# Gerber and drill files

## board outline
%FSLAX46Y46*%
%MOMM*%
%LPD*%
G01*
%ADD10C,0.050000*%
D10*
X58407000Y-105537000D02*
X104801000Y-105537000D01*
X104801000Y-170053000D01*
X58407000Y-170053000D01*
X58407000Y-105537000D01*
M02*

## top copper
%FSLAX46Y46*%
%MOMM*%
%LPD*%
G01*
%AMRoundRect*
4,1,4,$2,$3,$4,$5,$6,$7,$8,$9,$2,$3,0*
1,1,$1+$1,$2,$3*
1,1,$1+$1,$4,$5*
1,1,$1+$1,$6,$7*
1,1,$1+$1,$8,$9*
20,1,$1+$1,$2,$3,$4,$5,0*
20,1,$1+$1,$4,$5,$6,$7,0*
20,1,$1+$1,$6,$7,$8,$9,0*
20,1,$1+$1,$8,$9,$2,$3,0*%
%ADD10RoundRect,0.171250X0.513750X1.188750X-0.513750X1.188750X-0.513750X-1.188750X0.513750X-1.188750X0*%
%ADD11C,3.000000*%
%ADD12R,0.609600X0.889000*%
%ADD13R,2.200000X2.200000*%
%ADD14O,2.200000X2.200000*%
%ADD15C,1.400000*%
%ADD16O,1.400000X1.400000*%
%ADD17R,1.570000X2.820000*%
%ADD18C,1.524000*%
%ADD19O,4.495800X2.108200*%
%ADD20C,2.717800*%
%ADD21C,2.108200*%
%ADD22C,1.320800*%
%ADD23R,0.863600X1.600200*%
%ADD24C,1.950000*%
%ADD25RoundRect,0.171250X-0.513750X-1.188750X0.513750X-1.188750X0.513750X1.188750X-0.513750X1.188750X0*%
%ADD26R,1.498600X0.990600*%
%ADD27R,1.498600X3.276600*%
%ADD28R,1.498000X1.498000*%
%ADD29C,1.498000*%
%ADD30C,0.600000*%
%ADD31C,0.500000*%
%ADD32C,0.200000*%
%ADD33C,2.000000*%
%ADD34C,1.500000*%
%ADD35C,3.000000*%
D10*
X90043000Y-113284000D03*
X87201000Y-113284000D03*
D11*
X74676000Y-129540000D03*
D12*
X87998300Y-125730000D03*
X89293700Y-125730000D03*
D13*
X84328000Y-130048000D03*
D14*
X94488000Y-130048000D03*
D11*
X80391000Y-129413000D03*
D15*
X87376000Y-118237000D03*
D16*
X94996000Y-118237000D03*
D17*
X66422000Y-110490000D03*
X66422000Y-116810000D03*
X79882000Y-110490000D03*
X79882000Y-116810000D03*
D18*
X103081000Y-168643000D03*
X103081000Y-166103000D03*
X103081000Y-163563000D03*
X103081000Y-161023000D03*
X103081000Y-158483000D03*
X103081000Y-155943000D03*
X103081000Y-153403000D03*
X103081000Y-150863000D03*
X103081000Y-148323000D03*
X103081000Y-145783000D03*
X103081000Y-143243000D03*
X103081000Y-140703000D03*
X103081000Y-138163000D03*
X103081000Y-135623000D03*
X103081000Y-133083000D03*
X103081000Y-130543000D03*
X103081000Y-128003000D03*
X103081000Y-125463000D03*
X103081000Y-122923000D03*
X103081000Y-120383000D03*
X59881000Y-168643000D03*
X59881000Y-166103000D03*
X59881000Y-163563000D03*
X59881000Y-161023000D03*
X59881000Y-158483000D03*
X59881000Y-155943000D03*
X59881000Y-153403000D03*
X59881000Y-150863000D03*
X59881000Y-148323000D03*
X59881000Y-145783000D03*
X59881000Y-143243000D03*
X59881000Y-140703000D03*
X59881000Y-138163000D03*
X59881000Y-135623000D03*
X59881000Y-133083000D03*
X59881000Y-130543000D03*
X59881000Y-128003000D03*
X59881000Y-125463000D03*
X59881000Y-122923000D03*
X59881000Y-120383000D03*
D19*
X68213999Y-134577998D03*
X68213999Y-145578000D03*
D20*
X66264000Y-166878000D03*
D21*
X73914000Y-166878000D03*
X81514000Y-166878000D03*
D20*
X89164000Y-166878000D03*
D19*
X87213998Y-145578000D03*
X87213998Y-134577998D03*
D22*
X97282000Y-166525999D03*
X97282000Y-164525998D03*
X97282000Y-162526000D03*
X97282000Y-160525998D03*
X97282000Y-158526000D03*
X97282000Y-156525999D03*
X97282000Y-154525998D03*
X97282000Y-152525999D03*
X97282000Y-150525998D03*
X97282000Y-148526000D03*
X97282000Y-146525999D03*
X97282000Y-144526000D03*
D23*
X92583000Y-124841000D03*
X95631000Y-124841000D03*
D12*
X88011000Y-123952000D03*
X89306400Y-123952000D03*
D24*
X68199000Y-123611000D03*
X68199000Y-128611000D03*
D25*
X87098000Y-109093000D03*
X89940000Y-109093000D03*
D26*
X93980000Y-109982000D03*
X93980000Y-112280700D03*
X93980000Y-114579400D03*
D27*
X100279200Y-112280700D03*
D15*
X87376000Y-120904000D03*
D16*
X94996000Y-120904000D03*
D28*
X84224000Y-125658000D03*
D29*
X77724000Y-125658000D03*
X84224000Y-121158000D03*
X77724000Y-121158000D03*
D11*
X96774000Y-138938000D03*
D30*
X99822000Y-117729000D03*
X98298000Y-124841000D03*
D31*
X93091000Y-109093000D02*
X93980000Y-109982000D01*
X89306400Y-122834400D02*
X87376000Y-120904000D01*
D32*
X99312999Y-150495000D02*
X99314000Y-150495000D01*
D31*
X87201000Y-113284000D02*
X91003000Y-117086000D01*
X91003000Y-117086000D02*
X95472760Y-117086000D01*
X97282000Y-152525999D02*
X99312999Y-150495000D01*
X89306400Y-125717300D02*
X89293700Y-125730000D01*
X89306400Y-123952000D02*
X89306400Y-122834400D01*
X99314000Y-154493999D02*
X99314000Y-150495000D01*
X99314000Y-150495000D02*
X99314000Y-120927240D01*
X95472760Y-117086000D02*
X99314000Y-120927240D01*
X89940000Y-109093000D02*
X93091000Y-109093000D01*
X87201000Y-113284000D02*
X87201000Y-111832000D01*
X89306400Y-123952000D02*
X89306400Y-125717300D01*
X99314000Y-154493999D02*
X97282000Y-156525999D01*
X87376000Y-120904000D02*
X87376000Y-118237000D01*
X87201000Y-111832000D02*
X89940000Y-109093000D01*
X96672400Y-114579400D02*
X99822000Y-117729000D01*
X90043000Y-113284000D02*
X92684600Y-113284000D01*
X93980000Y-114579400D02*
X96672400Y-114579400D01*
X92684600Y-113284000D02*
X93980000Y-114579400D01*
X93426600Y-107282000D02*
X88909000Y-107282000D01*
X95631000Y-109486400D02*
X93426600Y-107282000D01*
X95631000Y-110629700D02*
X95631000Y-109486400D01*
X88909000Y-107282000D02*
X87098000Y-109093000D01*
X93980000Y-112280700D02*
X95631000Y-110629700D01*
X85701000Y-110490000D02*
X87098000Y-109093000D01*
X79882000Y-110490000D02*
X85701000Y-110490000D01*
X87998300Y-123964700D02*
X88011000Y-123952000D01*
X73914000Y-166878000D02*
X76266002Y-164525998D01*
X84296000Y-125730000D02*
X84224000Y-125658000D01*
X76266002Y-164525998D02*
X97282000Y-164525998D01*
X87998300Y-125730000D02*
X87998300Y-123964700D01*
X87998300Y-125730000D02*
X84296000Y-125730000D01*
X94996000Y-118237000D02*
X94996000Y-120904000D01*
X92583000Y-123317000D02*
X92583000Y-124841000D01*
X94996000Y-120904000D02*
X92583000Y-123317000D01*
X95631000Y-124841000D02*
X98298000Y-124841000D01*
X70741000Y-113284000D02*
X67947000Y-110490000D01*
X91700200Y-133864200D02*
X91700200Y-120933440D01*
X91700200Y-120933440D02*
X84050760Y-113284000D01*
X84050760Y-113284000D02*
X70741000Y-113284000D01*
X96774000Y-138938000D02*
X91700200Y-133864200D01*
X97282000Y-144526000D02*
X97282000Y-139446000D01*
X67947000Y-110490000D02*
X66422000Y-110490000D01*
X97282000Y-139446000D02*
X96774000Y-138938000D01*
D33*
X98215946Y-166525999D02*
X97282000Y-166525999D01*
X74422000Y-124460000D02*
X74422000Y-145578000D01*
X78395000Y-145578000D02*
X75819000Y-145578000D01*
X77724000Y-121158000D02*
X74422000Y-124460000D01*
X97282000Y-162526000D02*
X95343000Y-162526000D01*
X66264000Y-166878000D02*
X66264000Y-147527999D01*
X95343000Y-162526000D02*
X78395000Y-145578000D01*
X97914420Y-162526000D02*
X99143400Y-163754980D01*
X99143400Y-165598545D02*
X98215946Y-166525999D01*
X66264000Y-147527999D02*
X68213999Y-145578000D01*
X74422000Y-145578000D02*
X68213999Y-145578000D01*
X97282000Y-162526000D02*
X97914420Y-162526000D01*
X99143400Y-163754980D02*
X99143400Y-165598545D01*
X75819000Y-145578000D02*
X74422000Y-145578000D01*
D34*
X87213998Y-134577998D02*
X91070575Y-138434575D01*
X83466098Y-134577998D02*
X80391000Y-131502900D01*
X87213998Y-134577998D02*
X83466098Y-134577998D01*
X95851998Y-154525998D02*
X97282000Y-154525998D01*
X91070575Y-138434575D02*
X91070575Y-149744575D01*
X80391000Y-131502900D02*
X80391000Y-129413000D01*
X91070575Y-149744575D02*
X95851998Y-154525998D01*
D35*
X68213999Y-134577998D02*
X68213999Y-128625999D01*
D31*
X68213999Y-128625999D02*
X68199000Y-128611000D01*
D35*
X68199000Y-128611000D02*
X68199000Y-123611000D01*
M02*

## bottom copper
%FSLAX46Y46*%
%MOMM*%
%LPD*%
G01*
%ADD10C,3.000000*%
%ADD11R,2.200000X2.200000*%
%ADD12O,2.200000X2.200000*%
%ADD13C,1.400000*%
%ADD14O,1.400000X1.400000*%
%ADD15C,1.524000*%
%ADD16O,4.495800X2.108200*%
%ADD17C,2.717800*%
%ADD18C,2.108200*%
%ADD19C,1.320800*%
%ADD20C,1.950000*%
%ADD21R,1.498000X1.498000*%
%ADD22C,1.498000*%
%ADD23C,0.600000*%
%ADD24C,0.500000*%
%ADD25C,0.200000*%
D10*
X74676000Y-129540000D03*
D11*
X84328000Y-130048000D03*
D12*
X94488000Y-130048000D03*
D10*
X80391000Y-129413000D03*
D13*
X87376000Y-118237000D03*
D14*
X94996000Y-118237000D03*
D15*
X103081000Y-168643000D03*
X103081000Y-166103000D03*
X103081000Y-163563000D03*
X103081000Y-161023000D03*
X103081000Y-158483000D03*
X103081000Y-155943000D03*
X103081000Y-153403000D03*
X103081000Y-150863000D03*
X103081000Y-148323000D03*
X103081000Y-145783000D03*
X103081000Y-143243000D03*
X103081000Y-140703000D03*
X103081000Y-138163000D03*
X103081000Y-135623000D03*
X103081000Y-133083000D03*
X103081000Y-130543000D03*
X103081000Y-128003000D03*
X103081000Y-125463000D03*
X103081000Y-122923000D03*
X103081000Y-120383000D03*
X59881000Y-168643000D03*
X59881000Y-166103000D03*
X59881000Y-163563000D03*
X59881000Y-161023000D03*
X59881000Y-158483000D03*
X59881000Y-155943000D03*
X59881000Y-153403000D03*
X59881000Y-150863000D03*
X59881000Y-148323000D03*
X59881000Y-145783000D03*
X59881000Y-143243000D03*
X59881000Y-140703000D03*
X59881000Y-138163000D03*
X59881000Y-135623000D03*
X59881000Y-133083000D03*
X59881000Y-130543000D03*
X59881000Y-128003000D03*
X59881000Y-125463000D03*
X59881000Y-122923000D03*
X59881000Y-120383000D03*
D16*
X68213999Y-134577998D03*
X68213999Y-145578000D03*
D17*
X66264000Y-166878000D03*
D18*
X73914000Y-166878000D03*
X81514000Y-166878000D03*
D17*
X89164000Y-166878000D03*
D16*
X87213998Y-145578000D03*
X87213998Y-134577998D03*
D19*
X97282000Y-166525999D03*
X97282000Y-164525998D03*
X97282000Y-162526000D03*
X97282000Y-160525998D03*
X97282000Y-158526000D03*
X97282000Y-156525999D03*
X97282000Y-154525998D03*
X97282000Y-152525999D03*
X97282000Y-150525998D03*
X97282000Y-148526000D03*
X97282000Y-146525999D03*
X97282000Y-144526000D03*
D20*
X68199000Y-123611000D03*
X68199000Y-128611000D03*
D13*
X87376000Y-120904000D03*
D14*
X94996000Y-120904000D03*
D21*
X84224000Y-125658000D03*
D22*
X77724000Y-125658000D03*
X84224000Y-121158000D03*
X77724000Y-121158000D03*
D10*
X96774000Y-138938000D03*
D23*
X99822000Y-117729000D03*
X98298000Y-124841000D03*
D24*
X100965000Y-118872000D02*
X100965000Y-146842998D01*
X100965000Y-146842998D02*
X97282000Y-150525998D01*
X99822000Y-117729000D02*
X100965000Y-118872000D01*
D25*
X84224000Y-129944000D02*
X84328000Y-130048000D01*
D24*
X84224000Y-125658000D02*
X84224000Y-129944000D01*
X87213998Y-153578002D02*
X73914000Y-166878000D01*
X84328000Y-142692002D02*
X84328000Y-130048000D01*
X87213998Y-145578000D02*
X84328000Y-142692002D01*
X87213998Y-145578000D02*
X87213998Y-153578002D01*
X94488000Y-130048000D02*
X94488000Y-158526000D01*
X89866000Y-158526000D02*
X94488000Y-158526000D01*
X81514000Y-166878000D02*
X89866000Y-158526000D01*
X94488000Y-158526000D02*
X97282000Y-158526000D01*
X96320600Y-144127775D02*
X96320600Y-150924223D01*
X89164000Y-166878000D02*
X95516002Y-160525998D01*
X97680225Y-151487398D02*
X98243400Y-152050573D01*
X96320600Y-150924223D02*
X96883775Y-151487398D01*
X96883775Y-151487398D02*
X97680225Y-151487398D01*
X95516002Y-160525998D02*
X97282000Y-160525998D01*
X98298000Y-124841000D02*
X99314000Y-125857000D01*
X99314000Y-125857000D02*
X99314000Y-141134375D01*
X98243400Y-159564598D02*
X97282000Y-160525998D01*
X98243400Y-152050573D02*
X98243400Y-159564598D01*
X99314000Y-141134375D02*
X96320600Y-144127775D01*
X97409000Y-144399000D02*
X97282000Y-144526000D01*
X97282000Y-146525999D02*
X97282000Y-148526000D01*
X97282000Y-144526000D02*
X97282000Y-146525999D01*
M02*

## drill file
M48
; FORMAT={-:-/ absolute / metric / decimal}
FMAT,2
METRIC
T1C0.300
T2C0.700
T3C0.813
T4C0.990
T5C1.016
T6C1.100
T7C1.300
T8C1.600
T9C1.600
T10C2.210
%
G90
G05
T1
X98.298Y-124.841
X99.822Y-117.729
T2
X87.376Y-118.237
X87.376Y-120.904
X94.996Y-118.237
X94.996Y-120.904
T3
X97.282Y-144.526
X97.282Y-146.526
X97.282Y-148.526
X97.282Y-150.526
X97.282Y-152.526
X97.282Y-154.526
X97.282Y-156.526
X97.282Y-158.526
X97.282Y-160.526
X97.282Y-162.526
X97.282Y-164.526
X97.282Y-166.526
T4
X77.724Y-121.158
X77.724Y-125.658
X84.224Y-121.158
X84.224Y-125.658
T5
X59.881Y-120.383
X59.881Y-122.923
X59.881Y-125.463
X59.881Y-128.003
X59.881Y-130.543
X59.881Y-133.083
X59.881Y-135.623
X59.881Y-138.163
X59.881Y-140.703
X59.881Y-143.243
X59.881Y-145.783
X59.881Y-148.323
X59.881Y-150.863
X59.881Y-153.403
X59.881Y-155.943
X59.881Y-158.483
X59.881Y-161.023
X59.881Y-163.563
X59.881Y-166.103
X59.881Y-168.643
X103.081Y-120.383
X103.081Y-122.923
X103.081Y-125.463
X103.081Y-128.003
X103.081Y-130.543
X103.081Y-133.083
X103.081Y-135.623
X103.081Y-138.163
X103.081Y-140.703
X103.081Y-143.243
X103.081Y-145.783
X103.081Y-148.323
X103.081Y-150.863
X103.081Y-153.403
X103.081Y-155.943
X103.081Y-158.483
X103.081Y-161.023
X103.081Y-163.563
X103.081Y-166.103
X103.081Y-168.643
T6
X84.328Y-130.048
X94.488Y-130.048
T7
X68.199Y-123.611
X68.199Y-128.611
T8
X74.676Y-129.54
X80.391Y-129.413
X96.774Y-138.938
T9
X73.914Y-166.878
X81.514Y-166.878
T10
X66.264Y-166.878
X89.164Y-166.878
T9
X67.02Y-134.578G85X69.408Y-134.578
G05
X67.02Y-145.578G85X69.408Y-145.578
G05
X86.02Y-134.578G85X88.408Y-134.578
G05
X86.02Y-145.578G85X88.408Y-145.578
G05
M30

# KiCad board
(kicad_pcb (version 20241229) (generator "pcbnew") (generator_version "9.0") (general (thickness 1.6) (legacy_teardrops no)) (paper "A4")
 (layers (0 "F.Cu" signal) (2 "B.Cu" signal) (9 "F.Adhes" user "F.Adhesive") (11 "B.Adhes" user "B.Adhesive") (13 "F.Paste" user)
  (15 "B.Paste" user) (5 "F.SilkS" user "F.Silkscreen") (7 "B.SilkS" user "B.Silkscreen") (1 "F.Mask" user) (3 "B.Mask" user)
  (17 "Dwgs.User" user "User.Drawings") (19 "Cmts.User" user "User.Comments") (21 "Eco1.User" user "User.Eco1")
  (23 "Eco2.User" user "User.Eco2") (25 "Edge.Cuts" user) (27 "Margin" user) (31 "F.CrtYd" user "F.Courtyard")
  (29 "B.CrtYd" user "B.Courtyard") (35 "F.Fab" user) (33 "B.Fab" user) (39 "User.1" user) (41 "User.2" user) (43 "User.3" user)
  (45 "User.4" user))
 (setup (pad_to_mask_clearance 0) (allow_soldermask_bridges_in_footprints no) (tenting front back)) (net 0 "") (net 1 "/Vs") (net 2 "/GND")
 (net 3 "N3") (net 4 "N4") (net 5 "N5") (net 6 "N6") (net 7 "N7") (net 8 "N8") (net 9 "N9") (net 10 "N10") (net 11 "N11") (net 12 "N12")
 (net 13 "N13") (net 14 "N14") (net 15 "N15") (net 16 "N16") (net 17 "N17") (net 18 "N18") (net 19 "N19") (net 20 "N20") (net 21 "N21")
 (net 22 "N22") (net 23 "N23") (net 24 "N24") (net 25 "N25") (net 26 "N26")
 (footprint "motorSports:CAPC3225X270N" (layer "F.Cu") (at 88.622 113.284 180)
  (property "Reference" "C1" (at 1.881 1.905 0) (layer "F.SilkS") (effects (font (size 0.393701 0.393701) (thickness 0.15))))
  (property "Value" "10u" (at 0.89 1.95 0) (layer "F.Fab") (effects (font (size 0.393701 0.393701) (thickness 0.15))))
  (pad "1" smd roundrect (at -1.421 0 180) (size 1.37 2.72) (layers "F.Cu" "F.Mask" "F.Paste") (roundrect_rratio 0.125) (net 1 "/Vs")
   (solder_mask_margin 0.102))
  (pad "2" smd roundrect (at 1.421 0 180) (size 1.37 2.72) (layers "F.Cu" "F.Mask" "F.Paste") (roundrect_rratio 0.125) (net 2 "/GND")
   (solder_mask_margin 0.102)))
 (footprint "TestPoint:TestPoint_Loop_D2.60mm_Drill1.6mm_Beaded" (layer "F.Cu") (at 74.676 129.54)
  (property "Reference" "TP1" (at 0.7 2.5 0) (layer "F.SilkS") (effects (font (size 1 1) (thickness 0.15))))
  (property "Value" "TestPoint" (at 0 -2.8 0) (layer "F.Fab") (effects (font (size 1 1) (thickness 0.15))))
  (pad "1" thru_hole circle (at 0 0) (size 3 3) (drill 1.6) (layers "*.Cu" "*.Mask") (remove_unused_layers no) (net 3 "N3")))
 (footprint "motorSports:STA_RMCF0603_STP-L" (layer "F.Cu") (at 88.646 125.73)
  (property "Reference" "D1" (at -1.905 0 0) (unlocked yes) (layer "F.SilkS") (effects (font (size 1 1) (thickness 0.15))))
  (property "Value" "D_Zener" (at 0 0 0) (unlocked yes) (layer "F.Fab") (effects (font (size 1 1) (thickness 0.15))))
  (pad "1" smd rect (at -0.6477 0) (size 0.6096 0.889) (layers "F.Cu" "F.Mask" "F.Paste") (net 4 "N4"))
  (pad "2" smd rect (at 0.6477 0) (size 0.6096 0.889) (layers "F.Cu" "F.Mask" "F.Paste") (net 2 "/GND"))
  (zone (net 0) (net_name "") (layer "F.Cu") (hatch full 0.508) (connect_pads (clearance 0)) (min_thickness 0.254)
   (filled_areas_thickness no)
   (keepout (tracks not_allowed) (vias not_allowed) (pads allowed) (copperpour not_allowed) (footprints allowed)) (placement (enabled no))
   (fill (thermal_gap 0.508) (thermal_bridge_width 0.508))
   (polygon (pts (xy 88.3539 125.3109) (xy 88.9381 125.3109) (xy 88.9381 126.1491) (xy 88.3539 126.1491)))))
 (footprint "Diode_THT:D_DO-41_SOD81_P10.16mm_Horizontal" (layer "F.Cu") (at 84.328 130.048)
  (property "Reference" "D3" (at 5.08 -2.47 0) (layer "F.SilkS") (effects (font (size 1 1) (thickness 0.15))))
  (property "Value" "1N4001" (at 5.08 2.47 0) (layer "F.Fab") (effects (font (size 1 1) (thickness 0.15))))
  (pad "1" thru_hole rect (at 0 0) (size 2.2 2.2) (drill 1.1) (layers "*.Cu" "*.Mask") (remove_unused_layers no) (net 4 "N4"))
  (pad "2" thru_hole oval (at 10.16 0) (size 2.2 2.2) (drill 1.1) (layers "*.Cu" "*.Mask") (remove_unused_layers no) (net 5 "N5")))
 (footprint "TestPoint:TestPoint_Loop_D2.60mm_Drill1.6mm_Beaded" (layer "F.Cu") (at 80.391 129.413)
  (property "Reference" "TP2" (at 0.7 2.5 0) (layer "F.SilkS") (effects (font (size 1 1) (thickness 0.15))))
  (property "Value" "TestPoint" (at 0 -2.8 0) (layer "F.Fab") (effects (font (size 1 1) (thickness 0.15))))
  (pad "1" thru_hole circle (at 0 0) (size 3 3) (drill 1.6) (layers "*.Cu" "*.Mask") (remove_unused_layers no) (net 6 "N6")))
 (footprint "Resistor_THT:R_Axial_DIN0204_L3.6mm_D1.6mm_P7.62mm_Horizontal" (layer "F.Cu") (at 87.376 118.237)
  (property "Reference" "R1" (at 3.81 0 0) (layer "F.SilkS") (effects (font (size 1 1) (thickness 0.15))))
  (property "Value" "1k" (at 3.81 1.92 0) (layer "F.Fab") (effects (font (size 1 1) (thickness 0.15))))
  (pad "1" thru_hole circle (at 0 0) (size 1.4 1.4) (drill 0.7) (layers "*.Cu" "*.Mask") (remove_unused_layers no) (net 2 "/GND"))
  (pad "2" thru_hole oval (at 7.62 0) (size 1.4 1.4) (drill 0.7) (layers "*.Cu" "*.Mask") (remove_unused_layers no) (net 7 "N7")))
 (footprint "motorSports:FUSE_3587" (layer "F.Cu") (at 73.152 113.65)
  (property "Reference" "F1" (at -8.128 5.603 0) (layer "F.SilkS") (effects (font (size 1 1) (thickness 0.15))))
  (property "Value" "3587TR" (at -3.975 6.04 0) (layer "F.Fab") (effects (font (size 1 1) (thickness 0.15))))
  (pad "1_1" smd rect (at -6.73 -3.16) (size 1.57 2.82) (layers "F.Cu" "F.Mask" "F.Paste") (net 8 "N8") (solder_mask_margin 0.102))
  (pad "1_2" smd rect (at -6.73 3.16) (size 1.57 2.82) (layers "F.Cu" "F.Mask" "F.Paste") (solder_mask_margin 0.102))
  (pad "2_1" smd rect (at 6.73 -3.16) (size 1.57 2.82) (layers "F.Cu" "F.Mask" "F.Paste") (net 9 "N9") (solder_mask_margin 0.102))
  (pad "2_2" smd rect (at 6.73 3.16) (size 1.57 2.82) (layers "F.Cu" "F.Mask" "F.Paste") (solder_mask_margin 0.102)))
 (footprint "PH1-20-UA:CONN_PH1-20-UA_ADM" (layer "F.Cu") (at 103.081 168.643 90)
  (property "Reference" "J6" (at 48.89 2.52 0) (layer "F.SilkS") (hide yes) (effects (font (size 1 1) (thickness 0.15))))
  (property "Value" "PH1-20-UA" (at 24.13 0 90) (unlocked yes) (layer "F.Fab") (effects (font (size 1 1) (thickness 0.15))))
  (pad "1" thru_hole circle (at 0 0 90) (size 1.524 1.524) (drill 1.016) (layers "*.Cu" "*.Mask") (remove_unused_layers no))
  (pad "2" thru_hole circle (at 2.54 0 90) (size 1.524 1.524) (drill 1.016) (layers "*.Cu" "*.Mask") (remove_unused_layers no))
  (pad "3" thru_hole circle (at 5.08 0 90) (size 1.524 1.524) (drill 1.016) (layers "*.Cu" "*.Mask") (remove_unused_layers no))
  (pad "4" thru_hole circle (at 7.62 0 90) (size 1.524 1.524) (drill 1.016) (layers "*.Cu" "*.Mask") (remove_unused_layers no))
  (pad "5" thru_hole circle (at 10.16 0 90) (size 1.524 1.524) (drill 1.016) (layers "*.Cu" "*.Mask") (remove_unused_layers no))
  (pad "6" thru_hole circle (at 12.7 0 90) (size 1.524 1.524) (drill 1.016) (layers "*.Cu" "*.Mask") (remove_unused_layers no))
  (pad "7" thru_hole circle (at 15.24 0 90) (size 1.524 1.524) (drill 1.016) (layers "*.Cu" "*.Mask") (remove_unused_layers no))
  (pad "8" thru_hole circle (at 17.78 0 90) (size 1.524 1.524) (drill 1.016) (layers "*.Cu" "*.Mask") (remove_unused_layers no))
  (pad "9" thru_hole circle (at 20.32 0 90) (size 1.524 1.524) (drill 1.016) (layers "*.Cu" "*.Mask") (remove_unused_layers no))
  (pad "10" thru_hole circle (at 22.86 0 90) (size 1.524 1.524) (drill 1.016) (layers "*.Cu" "*.Mask") (remove_unused_layers no))
  (pad "11" thru_hole circle (at 25.4 0 90) (size 1.524 1.524) (drill 1.016) (layers "*.Cu" "*.Mask") (remove_unused_layers no))
  (pad "12" thru_hole circle (at 27.94 0 90) (size 1.524 1.524) (drill 1.016) (layers "*.Cu" "*.Mask") (remove_unused_layers no))
  (pad "13" thru_hole circle (at 30.48 0 90) (size 1.524 1.524) (drill 1.016) (layers "*.Cu" "*.Mask") (remove_unused_layers no))
  (pad "14" thru_hole circle (at 33.02 0 90) (size 1.524 1.524) (drill 1.016) (layers "*.Cu" "*.Mask") (remove_unused_layers no))
  (pad "15" thru_hole circle (at 35.56 0 90) (size 1.524 1.524) (drill 1.016) (layers "*.Cu" "*.Mask") (remove_unused_layers no))
  (pad "16" thru_hole circle (at 38.1 0 90) (size 1.524 1.524) (drill 1.016) (layers "*.Cu" "*.Mask") (remove_unused_layers no))
  (pad "17" thru_hole circle (at 40.64 0 90) (size 1.524 1.524) (drill 1.016) (layers "*.Cu" "*.Mask") (remove_unused_layers no))
  (pad "18" thru_hole circle (at 43.18 0 90) (size 1.524 1.524) (drill 1.016) (layers "*.Cu" "*.Mask") (remove_unused_layers no))
  (pad "19" thru_hole circle (at 45.72 0 90) (size 1.524 1.524) (drill 1.016) (layers "*.Cu" "*.Mask") (remove_unused_layers no))
  (pad "20" thru_hole circle (at 48.26 0 90) (size 1.524 1.524) (drill 1.016) (layers "*.Cu" "*.Mask") (remove_unused_layers no)))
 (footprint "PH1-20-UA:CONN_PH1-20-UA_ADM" (layer "F.Cu") (at 59.881 168.643 90)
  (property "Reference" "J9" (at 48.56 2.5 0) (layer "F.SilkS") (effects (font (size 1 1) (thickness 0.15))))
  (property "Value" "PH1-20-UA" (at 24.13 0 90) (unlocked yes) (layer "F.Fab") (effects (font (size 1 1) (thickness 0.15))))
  (pad "1" thru_hole circle (at 0 0 90) (size 1.524 1.524) (drill 1.016) (layers "*.Cu" "*.Mask") (remove_unused_layers no))
  (pad "2" thru_hole circle (at 2.54 0 90) (size 1.524 1.524) (drill 1.016) (layers "*.Cu" "*.Mask") (remove_unused_layers no))
  (pad "3" thru_hole circle (at 5.08 0 90) (size 1.524 1.524) (drill 1.016) (layers "*.Cu" "*.Mask") (remove_unused_layers no)
   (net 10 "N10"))
  (pad "4" thru_hole circle (at 7.62 0 90) (size 1.524 1.524) (drill 1.016) (layers "*.Cu" "*.Mask") (remove_unused_layers no))
  (pad "5" thru_hole circle (at 10.16 0 90) (size 1.524 1.524) (drill 1.016) (layers "*.Cu" "*.Mask") (remove_unused_layers no))
  (pad "6" thru_hole circle (at 12.7 0 90) (size 1.524 1.524) (drill 1.016) (layers "*.Cu" "*.Mask") (remove_unused_layers no))
  (pad "7" thru_hole circle (at 15.24 0 90) (size 1.524 1.524) (drill 1.016) (layers "*.Cu" "*.Mask") (remove_unused_layers no)
   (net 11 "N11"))
  (pad "8" thru_hole circle (at 17.78 0 90) (size 1.524 1.524) (drill 1.016) (layers "*.Cu" "*.Mask") (remove_unused_layers no)
   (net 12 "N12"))
  (pad "9" thru_hole circle (at 20.32 0 90) (size 1.524 1.524) (drill 1.016) (layers "*.Cu" "*.Mask") (remove_unused_layers no)
   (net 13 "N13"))
  (pad "10" thru_hole circle (at 22.86 0 90) (size 1.524 1.524) (drill 1.016) (layers "*.Cu" "*.Mask") (remove_unused_layers no)
   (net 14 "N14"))
  (pad "11" thru_hole circle (at 25.4 0 90) (size 1.524 1.524) (drill 1.016) (layers "*.Cu" "*.Mask") (remove_unused_layers no)
   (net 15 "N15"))
  (pad "12" thru_hole circle (at 27.94 0 90) (size 1.524 1.524) (drill 1.016) (layers "*.Cu" "*.Mask") (remove_unused_layers no)
   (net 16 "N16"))
  (pad "13" thru_hole circle (at 30.48 0 90) (size 1.524 1.524) (drill 1.016) (layers "*.Cu" "*.Mask") (remove_unused_layers no)
   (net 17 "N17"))
  (pad "14" thru_hole circle (at 33.02 0 90) (size 1.524 1.524) (drill 1.016) (layers "*.Cu" "*.Mask") (remove_unused_layers no)
   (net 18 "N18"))
  (pad "15" thru_hole circle (at 35.56 0 90) (size 1.524 1.524) (drill 1.016) (layers "*.Cu" "*.Mask") (remove_unused_layers no)
   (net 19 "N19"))
  (pad "16" thru_hole circle (at 38.1 0 90) (size 1.524 1.524) (drill 1.016) (layers "*.Cu" "*.Mask") (remove_unused_layers no)
   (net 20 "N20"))
  (pad "17" thru_hole circle (at 40.64 0 90) (size 1.524 1.524) (drill 1.016) (layers "*.Cu" "*.Mask") (remove_unused_layers no)
   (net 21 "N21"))
  (pad "18" thru_hole circle (at 43.18 0 90) (size 1.524 1.524) (drill 1.016) (layers "*.Cu" "*.Mask") (remove_unused_layers no)
   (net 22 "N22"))
  (pad "19" thru_hole circle (at 45.72 0 90) (size 1.524 1.524) (drill 1.016) (layers "*.Cu" "*.Mask") (remove_unused_layers no)
   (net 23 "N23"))
  (pad "20" thru_hole circle (at 48.26 0 90) (size 1.524 1.524) (drill 1.016) (layers "*.Cu" "*.Mask") (remove_unused_layers no)
   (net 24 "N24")))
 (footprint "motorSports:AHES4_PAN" (layer "F.Cu") (at 68.213999 134.577998)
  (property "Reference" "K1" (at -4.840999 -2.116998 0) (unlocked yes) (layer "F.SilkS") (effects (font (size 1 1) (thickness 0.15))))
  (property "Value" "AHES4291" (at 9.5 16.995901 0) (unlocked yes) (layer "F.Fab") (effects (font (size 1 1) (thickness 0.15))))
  (pad "1" thru_hole oval (at 0 0) (size 4.4958 2.1082) (drill oval 3.9878 1.6002) (layers "*.Cu" "*.Mask") (remove_unused_layers no)
   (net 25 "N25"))
  (pad "2" thru_hole oval (at 0 11.000002) (size 4.4958 2.1082) (drill oval 3.9878 1.6002) (layers "*.Cu" "*.Mask")
   (remove_unused_layers no) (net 3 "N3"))
  (pad "3" thru_hole circle (at -1.949999 32.300002) (size 2.7178 2.7178) (drill 2.2098) (layers "*.Cu" "*.Mask") (remove_unused_layers no)
   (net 3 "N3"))
  (pad "4" thru_hole circle (at 5.700001 32.300002) (size 2.1082 2.1082) (drill 1.6002) (layers "*.Cu" "*.Mask") (remove_unused_layers no)
   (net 4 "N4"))
  (pad "5" thru_hole circle (at 13.300001 32.300002) (size 2.1082 2.1082) (drill 1.6002) (layers "*.Cu" "*.Mask") (remove_unused_layers no)
   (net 5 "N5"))
  (pad "6" thru_hole circle (at 20.950001 32.300002) (size 2.7178 2.7178) (drill 2.2098) (layers "*.Cu" "*.Mask") (remove_unused_layers no)
   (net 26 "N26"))
  (pad "7" thru_hole oval (at 18.999999 11.000002) (size 4.4958 2.1082) (drill oval 3.9878 1.6002) (layers "*.Cu" "*.Mask")
   (remove_unused_layers no) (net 4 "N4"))
  (pad "8" thru_hole oval (at 18.999999 0) (size 4.4958 2.1082) (drill oval 3.9878 1.6002) (layers "*.Cu" "*.Mask")
   (remove_unused_layers no) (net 6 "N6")))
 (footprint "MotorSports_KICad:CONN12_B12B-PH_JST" (layer "F.Cu") (at 97.282 166.525999 90)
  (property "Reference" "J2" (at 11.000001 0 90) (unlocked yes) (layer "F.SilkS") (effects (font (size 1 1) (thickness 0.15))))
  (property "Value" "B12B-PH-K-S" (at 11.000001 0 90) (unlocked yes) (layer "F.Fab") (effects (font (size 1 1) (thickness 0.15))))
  (pad "1" thru_hole circle (at 0 0 90) (size 1.3208 1.3208) (drill 0.8128) (layers "*.Cu" "*.Mask") (remove_unused_layers no) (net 3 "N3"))
  (pad "2" thru_hole circle (at 2.000001 0 90) (size 1.3208 1.3208) (drill 0.8128) (layers "*.Cu" "*.Mask") (remove_unused_layers no)
   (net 4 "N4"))
  (pad "3" thru_hole circle (at 3.999999 0 90) (size 1.3208 1.3208) (drill 0.8128) (layers "*.Cu" "*.Mask") (remove_unused_layers no)
   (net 3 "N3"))
  (pad "4" thru_hole circle (at 6.000001 0 90) (size 1.3208 1.3208) (drill 0.8128) (layers "*.Cu" "*.Mask") (remove_unused_layers no)
   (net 26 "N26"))
  (pad "5" thru_hole circle (at 7.999999 0 90) (size 1.3208 1.3208) (drill 0.8128) (layers "*.Cu" "*.Mask") (remove_unused_layers no)
   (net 5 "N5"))
  (pad "6" thru_hole circle (at 10 0 90) (size 1.3208 1.3208) (drill 0.8128) (layers "*.Cu" "*.Mask") (remove_unused_layers no)
   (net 2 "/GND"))
  (pad "7" thru_hole circle (at 12.000001 0 90) (size 1.3208 1.3208) (drill 0.8128) (layers "*.Cu" "*.Mask") (remove_unused_layers no)
   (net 6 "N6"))
  (pad "8" thru_hole circle (at 14 0 90) (size 1.3208 1.3208) (drill 0.8128) (layers "*.Cu" "*.Mask") (remove_unused_layers no)
   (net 2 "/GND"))
  (pad "9" thru_hole circle (at 16.000001 0 90) (size 1.3208 1.3208) (drill 0.8128) (layers "*.Cu" "*.Mask") (remove_unused_layers no)
   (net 1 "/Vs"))
  (pad "10" thru_hole circle (at 17.999999 0 90) (size 1.3208 1.3208) (drill 0.8128) (layers "*.Cu" "*.Mask") (remove_unused_layers no)
   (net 8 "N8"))
  (pad "11" thru_hole circle (at 20 0 90) (size 1.3208 1.3208) (drill 0.8128) (layers "*.Cu" "*.Mask") (remove_unused_layers no)
   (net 8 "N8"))
  (pad "12" thru_hole circle (at 21.999999 0 90) (size 1.3208 1.3208) (drill 0.8128) (layers "*.Cu" "*.Mask") (remove_unused_layers no)
   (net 8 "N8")))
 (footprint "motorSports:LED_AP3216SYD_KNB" (layer "F.Cu") (at 94.107 124.841)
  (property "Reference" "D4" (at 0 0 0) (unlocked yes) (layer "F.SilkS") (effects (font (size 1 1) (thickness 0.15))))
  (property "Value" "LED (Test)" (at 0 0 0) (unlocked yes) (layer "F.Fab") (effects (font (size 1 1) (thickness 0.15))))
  (pad "1" smd rect (at -1.524 0) (size 0.8636 1.6002) (layers "F.Cu" "F.Mask" "F.Paste") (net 7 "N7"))
  (pad "2" smd rect (at 1.524 0) (size 0.8636 1.6002) (layers "F.Cu" "F.Mask" "F.Paste") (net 26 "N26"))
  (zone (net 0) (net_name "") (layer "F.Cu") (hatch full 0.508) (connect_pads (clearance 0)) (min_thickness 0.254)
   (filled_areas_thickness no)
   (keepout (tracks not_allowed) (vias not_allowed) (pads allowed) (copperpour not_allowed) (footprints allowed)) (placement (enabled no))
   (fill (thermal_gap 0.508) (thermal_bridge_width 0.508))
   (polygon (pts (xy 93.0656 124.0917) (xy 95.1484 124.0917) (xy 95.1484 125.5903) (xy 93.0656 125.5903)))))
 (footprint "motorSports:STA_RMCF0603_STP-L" (layer "F.Cu") (at 88.6587 123.952)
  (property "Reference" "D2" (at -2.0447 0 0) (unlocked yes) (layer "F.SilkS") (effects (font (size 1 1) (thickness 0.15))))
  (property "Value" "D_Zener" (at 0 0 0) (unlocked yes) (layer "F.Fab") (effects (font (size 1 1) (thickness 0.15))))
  (pad "1" smd rect (at -0.6477 0) (size 0.6096 0.889) (layers "F.Cu" "F.Mask" "F.Paste") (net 4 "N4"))
  (pad "2" smd rect (at 0.6477 0) (size 0.6096 0.889) (layers "F.Cu" "F.Mask" "F.Paste") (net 2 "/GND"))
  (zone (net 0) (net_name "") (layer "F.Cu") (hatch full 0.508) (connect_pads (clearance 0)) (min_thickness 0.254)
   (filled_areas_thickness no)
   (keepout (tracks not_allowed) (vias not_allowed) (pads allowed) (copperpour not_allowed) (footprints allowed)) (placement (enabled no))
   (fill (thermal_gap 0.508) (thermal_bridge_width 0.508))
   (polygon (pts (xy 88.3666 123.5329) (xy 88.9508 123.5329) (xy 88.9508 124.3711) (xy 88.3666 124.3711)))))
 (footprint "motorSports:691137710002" (layer "F.Cu") (at 68.199 126.111 -90)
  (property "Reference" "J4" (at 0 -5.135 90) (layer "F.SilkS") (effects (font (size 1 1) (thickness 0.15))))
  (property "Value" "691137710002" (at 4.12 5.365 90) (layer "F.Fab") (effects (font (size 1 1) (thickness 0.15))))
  (pad "1" thru_hole circle (at -2.5 0 270) (size 1.95 1.95) (drill 1.3) (layers "*.Cu" "*.Mask") (remove_unused_layers no) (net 25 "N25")
   (solder_mask_margin 0.102))
  (pad "2" thru_hole circle (at 2.5 0 270) (size 1.95 1.95) (drill 1.3) (layers "*.Cu" "*.Mask") (remove_unused_layers no) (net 25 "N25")
   (solder_mask_margin 0.102)))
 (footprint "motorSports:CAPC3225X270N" (layer "F.Cu") (at 88.519 109.093)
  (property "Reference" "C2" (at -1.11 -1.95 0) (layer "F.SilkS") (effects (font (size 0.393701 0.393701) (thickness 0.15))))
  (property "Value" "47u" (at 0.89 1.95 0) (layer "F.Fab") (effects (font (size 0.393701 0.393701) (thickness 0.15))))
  (pad "1" smd roundrect (at -1.421 0) (size 1.37 2.72) (layers "F.Cu" "F.Mask" "F.Paste") (roundrect_rratio 0.125) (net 9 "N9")
   (solder_mask_margin 0.102))
  (pad "2" smd roundrect (at 1.421 0) (size 1.37 2.72) (layers "F.Cu" "F.Mask" "F.Paste") (roundrect_rratio 0.125) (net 2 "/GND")
   (solder_mask_margin 0.102)))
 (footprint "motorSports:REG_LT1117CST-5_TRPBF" (layer "F.Cu") (at 97.1296 112.2807)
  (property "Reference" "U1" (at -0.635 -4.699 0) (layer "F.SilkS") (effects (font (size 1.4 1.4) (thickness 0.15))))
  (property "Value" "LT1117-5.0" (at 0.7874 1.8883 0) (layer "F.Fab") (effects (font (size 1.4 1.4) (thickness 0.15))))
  (pad "1" smd rect (at -3.1496 -2.2987) (size 1.4986 0.9906) (layers "F.Cu" "F.Mask" "F.Paste") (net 2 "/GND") (solder_mask_margin 0.102))
  (pad "2" smd rect (at -3.1496 0) (size 1.4986 0.9906) (layers "F.Cu" "F.Mask" "F.Paste") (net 9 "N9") (solder_mask_margin 0.102))
  (pad "3" smd rect (at -3.1496 2.2987) (size 1.4986 0.9906) (layers "F.Cu" "F.Mask" "F.Paste") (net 1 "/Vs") (solder_mask_margin 0.102))
  (pad "4" smd rect (at 3.1496 0) (size 1.4986 3.2766) (layers "F.Cu" "F.Mask" "F.Paste") (solder_mask_margin 0.102)))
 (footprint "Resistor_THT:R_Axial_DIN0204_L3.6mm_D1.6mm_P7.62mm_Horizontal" (layer "F.Cu") (at 87.376 120.904)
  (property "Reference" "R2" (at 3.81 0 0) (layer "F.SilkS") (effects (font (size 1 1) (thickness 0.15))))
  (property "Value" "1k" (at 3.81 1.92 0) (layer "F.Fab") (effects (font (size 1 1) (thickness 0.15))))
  (pad "1" thru_hole circle (at 0 0) (size 1.4 1.4) (drill 0.7) (layers "*.Cu" "*.Mask") (remove_unused_layers no) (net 2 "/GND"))
  (pad "2" thru_hole oval (at 7.62 0) (size 1.4 1.4) (drill 0.7) (layers "*.Cu" "*.Mask") (remove_unused_layers no) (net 7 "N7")))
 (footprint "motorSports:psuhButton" (layer "F.Cu") (at 80.974 123.408 180)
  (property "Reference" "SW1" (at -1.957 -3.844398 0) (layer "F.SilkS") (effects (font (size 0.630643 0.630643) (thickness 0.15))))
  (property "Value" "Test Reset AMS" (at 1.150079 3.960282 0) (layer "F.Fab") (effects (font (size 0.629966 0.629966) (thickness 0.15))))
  (pad "1" thru_hole rect (at -3.25 -2.25 180) (size 1.498 1.498) (drill 0.99) (layers "*.Cu" "*.Mask") (remove_unused_layers no)
   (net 4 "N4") (solder_mask_margin 0.102))
  (pad "2" thru_hole circle (at 3.25 -2.25 180) (size 1.498 1.498) (drill 0.99) (layers "*.Cu" "*.Mask") (remove_unused_layers no)
   (solder_mask_margin 0.102))
  (pad "3" thru_hole circle (at -3.25 2.25 180) (size 1.498 1.498) (drill 0.99) (layers "*.Cu" "*.Mask") (remove_unused_layers no)
   (solder_mask_margin 0.102))
  (pad "4" thru_hole circle (at 3.25 2.25 180) (size 1.498 1.498) (drill 0.99) (layers "*.Cu" "*.Mask") (remove_unused_layers no)
   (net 3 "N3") (solder_mask_margin 0.102)))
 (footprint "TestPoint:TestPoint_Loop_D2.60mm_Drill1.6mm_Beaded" (layer "F.Cu") (at 96.774 138.938)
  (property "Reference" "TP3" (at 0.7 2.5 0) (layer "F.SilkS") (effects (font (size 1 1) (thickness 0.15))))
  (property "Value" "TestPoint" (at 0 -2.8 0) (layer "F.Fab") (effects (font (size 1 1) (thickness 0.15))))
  (pad "1" thru_hole circle (at 0 0) (size 3 3) (drill 1.6) (layers "*.Cu" "*.Mask") (remove_unused_layers no) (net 8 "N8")))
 (gr_rect (start 58.407 105.537) (end 104.801 170.053) (stroke (width 0.05) (type default)) (fill no) (layer "Edge.Cuts"))
 (segment (start 93.091 109.093) (end 93.98 109.982) (width 0.5) (layer "F.Cu") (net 2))
 (segment (start 89.3064 122.8344) (end 87.376 120.904) (width 0.5) (layer "F.Cu") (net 2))
 (segment (start 99.312999 150.495) (end 99.314 150.495) (width 0.2) (layer "F.Cu") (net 2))
 (segment (start 87.201 113.284) (end 91.003 117.086) (width 0.5) (layer "F.Cu") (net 2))
 (segment (start 91.003 117.086) (end 95.47276 117.086) (width 0.5) (layer "F.Cu") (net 2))
 (segment (start 97.282 152.525999) (end 99.312999 150.495) (width 0.5) (layer "F.Cu") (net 2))
 (segment (start 89.3064 125.7173) (end 89.2937 125.73) (width 0.5) (layer "F.Cu") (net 2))
 (segment (start 89.3064 123.952) (end 89.3064 122.8344) (width 0.5) (layer "F.Cu") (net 2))
 (segment (start 99.314 154.493999) (end 99.314 150.495) (width 0.5) (layer "F.Cu") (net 2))
 (segment (start 99.314 150.495) (end 99.314 120.92724) (width 0.5) (layer "F.Cu") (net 2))
 (segment (start 95.47276 117.086) (end 99.314 120.92724) (width 0.5) (layer "F.Cu") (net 2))
 (segment (start 89.94 109.093) (end 93.091 109.093) (width 0.5) (layer "F.Cu") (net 2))
 (segment (start 87.201 113.284) (end 87.201 111.832) (width 0.5) (layer "F.Cu") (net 2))
 (segment (start 89.3064 123.952) (end 89.3064 125.7173) (width 0.5) (layer "F.Cu") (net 2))
 (segment (start 99.314 154.493999) (end 97.282 156.525999) (width 0.5) (layer "F.Cu") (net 2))
 (segment (start 87.376 120.904) (end 87.376 118.237) (width 0.5) (layer "F.Cu") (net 2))
 (segment (start 87.201 111.832) (end 89.94 109.093) (width 0.5) (layer "F.Cu") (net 2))
 (segment (start 96.6724 114.5794) (end 99.822 117.729) (width 0.5) (layer "F.Cu") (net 1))
 (segment (start 90.043 113.284) (end 92.6846 113.284) (width 0.5) (layer "F.Cu") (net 1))
 (segment (start 93.98 114.5794) (end 96.6724 114.5794) (width 0.5) (layer "F.Cu") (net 1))
 (segment (start 92.6846 113.284) (end 93.98 114.5794) (width 0.5) (layer "F.Cu") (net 1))
 (via (at 99.822 117.729) (size 0.6) (drill 0.3) (layers "F.Cu" "B.Cu") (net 1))
 (segment (start 100.965 118.872) (end 100.965 146.842998) (width 0.5) (layer "B.Cu") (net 1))
 (segment (start 100.965 146.842998) (end 97.282 150.525998) (width 0.5) (layer "B.Cu") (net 1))
 (segment (start 99.822 117.729) (end 100.965 118.872) (width 0.5) (layer "B.Cu") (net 1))
 (segment (start 93.4266 107.282) (end 88.909 107.282) (width 0.5) (layer "F.Cu") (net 9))
 (segment (start 95.631 109.4864) (end 93.4266 107.282) (width 0.5) (layer "F.Cu") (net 9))
 (segment (start 95.631 110.6297) (end 95.631 109.4864) (width 0.5) (layer "F.Cu") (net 9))
 (segment (start 88.909 107.282) (end 87.098 109.093) (width 0.5) (layer "F.Cu") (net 9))
 (segment (start 93.98 112.2807) (end 95.631 110.6297) (width 0.5) (layer "F.Cu") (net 9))
 (segment (start 85.701 110.49) (end 87.098 109.093) (width 0.5) (layer "F.Cu") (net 9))
 (segment (start 79.882 110.49) (end 85.701 110.49) (width 0.5) (layer "F.Cu") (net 9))
 (segment (start 87.9983 123.9647) (end 88.011 123.952) (width 0.5) (layer "F.Cu") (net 4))
 (segment (start 73.914 166.878) (end 76.266002 164.525998) (width 0.5) (layer "F.Cu") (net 4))
 (segment (start 84.296 125.73) (end 84.224 125.658) (width 0.5) (layer "F.Cu") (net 4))
 (segment (start 76.266002 164.525998) (end 97.282 164.525998) (width 0.5) (layer "F.Cu") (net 4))
 (segment (start 87.9983 125.73) (end 87.9983 123.9647) (width 0.5) (layer "F.Cu") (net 4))
 (segment (start 87.9983 125.73) (end 84.296 125.73) (width 0.5) (layer "F.Cu") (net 4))
 (segment (start 84.224 129.944) (end 84.328 130.048) (width 0.2) (layer "B.Cu") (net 4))
 (segment (start 84.224 125.658) (end 84.224 129.944) (width 0.5) (layer "B.Cu") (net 4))
 (segment (start 87.213998 153.578002) (end 73.914 166.878) (width 0.5) (layer "B.Cu") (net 4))
 (segment (start 84.328 142.692002) (end 84.328 130.048) (width 0.5) (layer "B.Cu") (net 4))
 (segment (start 87.213998 145.578) (end 84.328 142.692002) (width 0.5) (layer "B.Cu") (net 4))
 (segment (start 87.213998 145.578) (end 87.213998 153.578002) (width 0.5) (layer "B.Cu") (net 4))
 (segment (start 94.488 130.048) (end 94.488 158.526) (width 0.5) (layer "B.Cu") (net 5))
 (segment (start 89.866 158.526) (end 94.488 158.526) (width 0.5) (layer "B.Cu") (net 5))
 (segment (start 81.514 166.878) (end 89.866 158.526) (width 0.5) (layer "B.Cu") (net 5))
 (segment (start 94.488 158.526) (end 97.282 158.526) (width 0.5) (layer "B.Cu") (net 5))
 (segment (start 94.996 118.237) (end 94.996 120.904) (width 0.5) (layer "F.Cu") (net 7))
 (segment (start 92.583 123.317) (end 92.583 124.841) (width 0.5) (layer "F.Cu") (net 7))
 (segment (start 94.996 120.904) (end 92.583 123.317) (width 0.5) (layer "F.Cu") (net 7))
 (segment (start 95.631 124.841) (end 98.298 124.841) (width 0.5) (layer "F.Cu") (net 26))
 (via (at 98.298 124.841) (size 0.6) (drill 0.3) (layers "F.Cu" "B.Cu") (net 26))
 (segment (start 96.3206 144.127775) (end 96.3206 150.924223) (width 0.5) (layer "B.Cu") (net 26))
 (segment (start 89.164 166.878) (end 95.516002 160.525998) (width 0.5) (layer "B.Cu") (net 26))
 (segment (start 97.680225 151.487398) (end 98.2434 152.050573) (width 0.5) (layer "B.Cu") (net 26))
 (segment (start 96.3206 150.924223) (end 96.883775 151.487398) (width 0.5) (layer "B.Cu") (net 26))
 (segment (start 96.883775 151.487398) (end 97.680225 151.487398) (width 0.5) (layer "B.Cu") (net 26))
 (segment (start 95.516002 160.525998) (end 97.282 160.525998) (width 0.5) (layer "B.Cu") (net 26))
 (segment (start 98.298 124.841) (end 99.314 125.857) (width 0.5) (layer "B.Cu") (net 26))
 (segment (start 99.314 125.857) (end 99.314 141.134375) (width 0.5) (layer "B.Cu") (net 26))
 (segment (start 98.2434 159.564598) (end 97.282 160.525998) (width 0.5) (layer "B.Cu") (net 26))
 (segment (start 98.2434 152.050573) (end 98.2434 159.564598) (width 0.5) (layer "B.Cu") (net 26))
 (segment (start 99.314 141.134375) (end 96.3206 144.127775) (width 0.5) (layer "B.Cu") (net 26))
 (segment (start 70.741 113.284) (end 67.947 110.49) (width 0.5) (layer "F.Cu") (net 8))
 (segment (start 91.7002 133.8642) (end 91.7002 120.93344) (width 0.5) (layer "F.Cu") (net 8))
 (segment (start 91.7002 120.93344) (end 84.05076 113.284) (width 0.5) (layer "F.Cu") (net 8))
 (segment (start 84.05076 113.284) (end 70.741 113.284) (width 0.5) (layer "F.Cu") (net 8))
 (segment (start 96.774 138.938) (end 91.7002 133.8642) (width 0.5) (layer "F.Cu") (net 8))
 (segment (start 97.282 144.526) (end 97.282 139.446) (width 0.5) (layer "F.Cu") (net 8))
 (segment (start 67.947 110.49) (end 66.422 110.49) (width 0.5) (layer "F.Cu") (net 8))
 (segment (start 97.282 139.446) (end 96.774 138.938) (width 0.5) (layer "F.Cu") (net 8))
 (segment (start 97.409 144.399) (end 97.282 144.526) (width 0.5) (layer "B.Cu") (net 8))
 (segment (start 97.282 146.525999) (end 97.282 148.526) (width 0.5) (layer "B.Cu") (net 8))
 (segment (start 97.282 144.526) (end 97.282 146.525999) (width 0.5) (layer "B.Cu") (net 8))
 (segment (start 98.215946 166.525999) (end 97.282 166.525999) (width 2) (layer "F.Cu") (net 3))
 (segment (start 74.422 124.46) (end 74.422 145.578) (width 2) (layer "F.Cu") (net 3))
 (segment (start 78.395 145.578) (end 75.819 145.578) (width 2) (layer "F.Cu") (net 3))
 (segment (start 77.724 121.158) (end 74.422 124.46) (width 2) (layer "F.Cu") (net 3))
 (segment (start 97.282 162.526) (end 95.343 162.526) (width 2) (layer "F.Cu") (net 3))
 (segment (start 66.264 166.878) (end 66.264 147.527999) (width 2) (layer "F.Cu") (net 3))
 (segment (start 95.343 162.526) (end 78.395 145.578) (width 2) (layer "F.Cu") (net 3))
 (segment (start 97.91442 162.526) (end 99.1434 163.75498) (width 2) (layer "F.Cu") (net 3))
 (segment (start 99.1434 165.598545) (end 98.215946 166.525999) (width 2) (layer "F.Cu") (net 3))
 (segment (start 66.264 147.527999) (end 68.213999 145.578) (width 2) (layer "F.Cu") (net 3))
 (segment (start 74.422 145.578) (end 68.213999 145.578) (width 2) (layer "F.Cu") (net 3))
 (segment (start 97.282 162.526) (end 97.91442 162.526) (width 2) (layer "F.Cu") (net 3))
 (segment (start 99.1434 163.75498) (end 99.1434 165.598545) (width 2) (layer "F.Cu") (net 3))
 (segment (start 75.819 145.578) (end 74.422 145.578) (width 2) (layer "F.Cu") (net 3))
 (segment (start 87.213998 134.577998) (end 91.070575 138.434575) (width 1.5) (layer "F.Cu") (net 6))
 (segment (start 83.466098 134.577998) (end 80.391 131.5029) (width 1.5) (layer "F.Cu") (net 6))
 (segment (start 87.213998 134.577998) (end 83.466098 134.577998) (width 1.5) (layer "F.Cu") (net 6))
 (segment (start 95.851998 154.525998) (end 97.282 154.525998) (width 1.5) (layer "F.Cu") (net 6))
 (segment (start 91.070575 138.434575) (end 91.070575 149.744575) (width 1.5) (layer "F.Cu") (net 6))
 (segment (start 80.391 131.5029) (end 80.391 129.413) (width 1.5) (layer "F.Cu") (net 6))
 (segment (start 91.070575 149.744575) (end 95.851998 154.525998) (width 1.5) (layer "F.Cu") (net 6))
 (segment (start 68.213999 134.577998) (end 68.213999 128.625999) (width 3) (layer "F.Cu") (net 25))
 (segment (start 68.213999 128.625999) (end 68.199 128.611) (width 0.5) (layer "F.Cu") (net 25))
 (segment (start 68.199 128.611) (end 68.199 123.611) (width 3) (layer "F.Cu") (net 25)))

